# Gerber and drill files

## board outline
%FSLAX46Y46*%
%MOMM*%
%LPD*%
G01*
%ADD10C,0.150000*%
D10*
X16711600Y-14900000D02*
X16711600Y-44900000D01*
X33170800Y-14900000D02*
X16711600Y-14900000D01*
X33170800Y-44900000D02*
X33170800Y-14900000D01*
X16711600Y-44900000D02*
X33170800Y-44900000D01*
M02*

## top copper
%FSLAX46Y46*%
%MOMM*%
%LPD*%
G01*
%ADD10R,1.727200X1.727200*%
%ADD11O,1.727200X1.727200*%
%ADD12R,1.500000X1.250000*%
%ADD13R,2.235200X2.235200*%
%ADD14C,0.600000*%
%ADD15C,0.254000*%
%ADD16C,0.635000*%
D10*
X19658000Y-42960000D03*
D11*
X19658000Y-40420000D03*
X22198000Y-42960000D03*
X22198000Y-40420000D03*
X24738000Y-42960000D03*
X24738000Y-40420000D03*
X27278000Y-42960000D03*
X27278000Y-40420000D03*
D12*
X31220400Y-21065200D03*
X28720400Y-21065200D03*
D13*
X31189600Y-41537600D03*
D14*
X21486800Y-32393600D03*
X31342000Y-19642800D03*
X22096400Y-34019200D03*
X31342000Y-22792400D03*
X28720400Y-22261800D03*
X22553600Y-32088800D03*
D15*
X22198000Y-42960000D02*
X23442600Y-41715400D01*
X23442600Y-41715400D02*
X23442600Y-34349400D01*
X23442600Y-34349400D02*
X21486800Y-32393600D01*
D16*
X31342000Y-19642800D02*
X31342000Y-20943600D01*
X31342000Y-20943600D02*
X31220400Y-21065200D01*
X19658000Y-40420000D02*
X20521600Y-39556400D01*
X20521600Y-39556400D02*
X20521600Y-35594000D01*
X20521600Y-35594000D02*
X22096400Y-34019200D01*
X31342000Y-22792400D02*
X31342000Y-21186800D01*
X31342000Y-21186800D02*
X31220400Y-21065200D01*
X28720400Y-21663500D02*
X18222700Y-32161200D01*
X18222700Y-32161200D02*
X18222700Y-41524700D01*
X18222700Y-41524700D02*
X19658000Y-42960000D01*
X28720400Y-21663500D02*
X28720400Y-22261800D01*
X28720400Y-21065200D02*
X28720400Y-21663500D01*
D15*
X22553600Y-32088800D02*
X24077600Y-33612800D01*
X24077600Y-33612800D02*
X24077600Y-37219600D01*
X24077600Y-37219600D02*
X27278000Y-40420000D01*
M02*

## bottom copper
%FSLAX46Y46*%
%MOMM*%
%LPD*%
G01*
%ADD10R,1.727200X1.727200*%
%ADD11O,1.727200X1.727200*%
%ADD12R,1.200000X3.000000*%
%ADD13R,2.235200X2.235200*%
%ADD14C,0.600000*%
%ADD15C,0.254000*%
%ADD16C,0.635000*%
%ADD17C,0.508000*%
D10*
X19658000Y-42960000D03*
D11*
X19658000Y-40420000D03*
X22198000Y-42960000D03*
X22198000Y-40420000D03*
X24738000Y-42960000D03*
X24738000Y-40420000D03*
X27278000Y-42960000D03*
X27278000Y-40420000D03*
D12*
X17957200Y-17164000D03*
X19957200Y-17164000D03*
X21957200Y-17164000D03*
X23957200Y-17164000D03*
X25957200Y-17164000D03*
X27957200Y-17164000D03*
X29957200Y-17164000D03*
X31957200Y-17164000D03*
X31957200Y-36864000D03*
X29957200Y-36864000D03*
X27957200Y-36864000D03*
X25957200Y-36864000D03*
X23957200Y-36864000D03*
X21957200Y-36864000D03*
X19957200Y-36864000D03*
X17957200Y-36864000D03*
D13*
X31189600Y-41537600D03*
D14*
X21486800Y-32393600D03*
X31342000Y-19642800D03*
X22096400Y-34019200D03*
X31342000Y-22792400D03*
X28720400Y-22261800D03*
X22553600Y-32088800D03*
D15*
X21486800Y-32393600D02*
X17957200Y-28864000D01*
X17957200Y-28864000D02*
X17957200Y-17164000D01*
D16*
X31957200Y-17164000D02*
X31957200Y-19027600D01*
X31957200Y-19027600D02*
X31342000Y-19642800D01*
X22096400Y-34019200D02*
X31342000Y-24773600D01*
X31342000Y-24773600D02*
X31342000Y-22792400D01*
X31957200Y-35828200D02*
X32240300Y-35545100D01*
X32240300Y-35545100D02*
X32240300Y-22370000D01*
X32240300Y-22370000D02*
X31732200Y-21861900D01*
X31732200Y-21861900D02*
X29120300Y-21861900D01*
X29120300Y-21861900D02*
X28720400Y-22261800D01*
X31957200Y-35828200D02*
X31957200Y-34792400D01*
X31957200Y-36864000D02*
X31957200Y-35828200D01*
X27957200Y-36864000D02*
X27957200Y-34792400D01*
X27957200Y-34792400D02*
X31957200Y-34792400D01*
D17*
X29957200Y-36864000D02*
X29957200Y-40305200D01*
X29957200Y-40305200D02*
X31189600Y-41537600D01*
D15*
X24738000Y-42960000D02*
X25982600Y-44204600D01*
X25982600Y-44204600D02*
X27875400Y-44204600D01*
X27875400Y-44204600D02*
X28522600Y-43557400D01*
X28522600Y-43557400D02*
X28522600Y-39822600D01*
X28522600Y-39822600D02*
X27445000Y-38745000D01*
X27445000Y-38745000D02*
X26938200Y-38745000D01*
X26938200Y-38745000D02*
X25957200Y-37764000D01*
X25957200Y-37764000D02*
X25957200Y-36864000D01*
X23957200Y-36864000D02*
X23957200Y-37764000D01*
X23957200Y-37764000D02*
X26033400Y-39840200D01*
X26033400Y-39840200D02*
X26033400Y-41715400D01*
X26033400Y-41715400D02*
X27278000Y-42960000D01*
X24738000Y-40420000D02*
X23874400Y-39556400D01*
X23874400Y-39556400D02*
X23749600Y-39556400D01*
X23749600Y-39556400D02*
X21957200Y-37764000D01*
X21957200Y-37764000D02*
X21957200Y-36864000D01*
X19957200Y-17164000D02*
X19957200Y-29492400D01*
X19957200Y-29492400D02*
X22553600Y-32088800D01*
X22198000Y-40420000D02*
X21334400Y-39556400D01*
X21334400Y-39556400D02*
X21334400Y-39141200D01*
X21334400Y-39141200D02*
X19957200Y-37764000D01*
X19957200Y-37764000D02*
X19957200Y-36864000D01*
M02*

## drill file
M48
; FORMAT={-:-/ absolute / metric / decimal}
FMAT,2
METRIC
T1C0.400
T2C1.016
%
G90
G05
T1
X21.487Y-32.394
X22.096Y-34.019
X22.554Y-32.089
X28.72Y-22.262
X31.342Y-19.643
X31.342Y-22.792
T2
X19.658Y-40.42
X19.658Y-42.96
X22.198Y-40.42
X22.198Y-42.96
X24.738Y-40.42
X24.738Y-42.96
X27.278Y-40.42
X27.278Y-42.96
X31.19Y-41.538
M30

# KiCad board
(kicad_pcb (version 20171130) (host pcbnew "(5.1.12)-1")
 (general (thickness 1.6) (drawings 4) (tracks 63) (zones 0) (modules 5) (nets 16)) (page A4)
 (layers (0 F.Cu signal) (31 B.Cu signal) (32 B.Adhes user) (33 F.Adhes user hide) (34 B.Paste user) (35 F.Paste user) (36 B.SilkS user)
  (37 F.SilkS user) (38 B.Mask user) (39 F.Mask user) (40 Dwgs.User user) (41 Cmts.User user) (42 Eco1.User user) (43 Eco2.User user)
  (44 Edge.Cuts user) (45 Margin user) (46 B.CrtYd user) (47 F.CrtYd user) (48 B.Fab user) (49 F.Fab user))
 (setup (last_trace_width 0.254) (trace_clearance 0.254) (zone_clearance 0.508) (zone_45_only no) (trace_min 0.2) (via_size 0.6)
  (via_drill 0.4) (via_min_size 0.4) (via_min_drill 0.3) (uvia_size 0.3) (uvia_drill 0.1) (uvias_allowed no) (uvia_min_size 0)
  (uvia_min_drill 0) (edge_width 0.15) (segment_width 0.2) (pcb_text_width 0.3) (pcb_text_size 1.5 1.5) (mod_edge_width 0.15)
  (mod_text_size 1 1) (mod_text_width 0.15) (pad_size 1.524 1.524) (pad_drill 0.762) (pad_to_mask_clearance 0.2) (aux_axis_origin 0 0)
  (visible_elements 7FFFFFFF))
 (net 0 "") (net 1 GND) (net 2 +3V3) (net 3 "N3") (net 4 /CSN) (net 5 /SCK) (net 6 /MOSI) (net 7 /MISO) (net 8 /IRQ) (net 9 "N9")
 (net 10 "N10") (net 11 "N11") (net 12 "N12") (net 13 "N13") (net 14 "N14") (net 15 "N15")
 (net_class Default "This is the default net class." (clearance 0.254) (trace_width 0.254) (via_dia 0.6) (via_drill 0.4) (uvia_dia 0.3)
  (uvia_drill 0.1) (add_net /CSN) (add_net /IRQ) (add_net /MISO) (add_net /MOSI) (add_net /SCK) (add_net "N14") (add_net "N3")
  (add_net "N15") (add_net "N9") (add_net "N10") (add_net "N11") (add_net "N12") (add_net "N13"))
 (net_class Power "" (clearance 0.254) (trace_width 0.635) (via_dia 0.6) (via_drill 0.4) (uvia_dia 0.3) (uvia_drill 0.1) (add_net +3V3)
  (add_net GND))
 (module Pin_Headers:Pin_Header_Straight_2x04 (layer F.Cu) (at 19.658 42.96 90)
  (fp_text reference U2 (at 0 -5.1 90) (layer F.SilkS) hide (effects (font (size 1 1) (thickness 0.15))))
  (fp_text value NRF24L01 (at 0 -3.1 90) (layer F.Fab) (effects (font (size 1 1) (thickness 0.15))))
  (pad 1 thru_hole rect (at 0 0 90) (size 1.7272 1.7272) (drill 1.016) (layers *.Cu *.Mask F.SilkS) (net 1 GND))
  (pad 2 thru_hole oval (at 2.54 0 90) (size 1.7272 1.7272) (drill 1.016) (layers *.Cu *.Mask F.SilkS) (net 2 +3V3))
  (pad 3 thru_hole oval (at 0 2.54 90) (size 1.7272 1.7272) (drill 1.016) (layers *.Cu *.Mask F.SilkS) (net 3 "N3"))
  (pad 4 thru_hole oval (at 2.54 2.54 90) (size 1.7272 1.7272) (drill 1.016) (layers *.Cu *.Mask F.SilkS) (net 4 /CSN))
  (pad 5 thru_hole oval (at 0 5.08 90) (size 1.7272 1.7272) (drill 1.016) (layers *.Cu *.Mask F.SilkS) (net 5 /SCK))
  (pad 6 thru_hole oval (at 2.54 5.08 90) (size 1.7272 1.7272) (drill 1.016) (layers *.Cu *.Mask F.SilkS) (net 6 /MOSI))
  (pad 7 thru_hole oval (at 0 7.62 90) (size 1.7272 1.7272) (drill 1.016) (layers *.Cu *.Mask F.SilkS) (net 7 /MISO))
  (pad 8 thru_hole oval (at 2.54 7.62 90) (size 1.7272 1.7272) (drill 1.016) (layers *.Cu *.Mask F.SilkS) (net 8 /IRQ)))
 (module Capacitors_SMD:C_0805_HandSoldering (layer F.Cu) (at 29.9704 21.0652 180)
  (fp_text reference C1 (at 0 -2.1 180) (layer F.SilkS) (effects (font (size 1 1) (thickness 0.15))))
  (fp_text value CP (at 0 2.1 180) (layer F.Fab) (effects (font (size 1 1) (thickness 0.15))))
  (pad 1 smd rect (at -1.25 0 180) (size 1.5 1.25) (layers F.Cu F.Paste F.Mask) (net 2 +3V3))
  (pad 2 smd rect (at 1.25 0 180) (size 1.5 1.25) (layers F.Cu F.Paste F.Mask) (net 1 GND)))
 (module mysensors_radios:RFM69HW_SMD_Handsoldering (layer B.Cu) (at 17.9572 18.564 270)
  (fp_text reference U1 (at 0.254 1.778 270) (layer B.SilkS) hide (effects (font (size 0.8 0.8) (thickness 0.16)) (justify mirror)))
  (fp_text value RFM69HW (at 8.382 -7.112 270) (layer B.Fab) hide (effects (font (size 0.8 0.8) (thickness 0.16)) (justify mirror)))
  (pad 1 smd rect (at -1.4 0 270) (size 3 1.2) (layers B.Cu B.Paste B.Mask) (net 3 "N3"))
  (pad 2 smd rect (at -1.4 -2 270) (size 3 1.2) (layers B.Cu B.Paste B.Mask) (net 8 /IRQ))
  (pad 3 smd rect (at -1.4 -4 270) (size 3 1.2) (layers B.Cu B.Paste B.Mask) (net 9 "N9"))
  (pad 4 smd rect (at -1.4 -6 270) (size 3 1.2) (layers B.Cu B.Paste B.Mask) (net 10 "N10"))
  (pad 5 smd rect (at -1.4 -8 270) (size 3 1.2) (layers B.Cu B.Paste B.Mask) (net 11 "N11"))
  (pad 6 smd rect (at -1.4 -10 270) (size 3 1.2) (layers B.Cu B.Paste B.Mask) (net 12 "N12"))
  (pad 7 smd rect (at -1.4 -12 270) (size 3 1.2) (layers B.Cu B.Paste B.Mask) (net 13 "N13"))
  (pad 8 smd rect (at -1.4 -14 270) (size 3 1.2) (layers B.Cu B.Paste B.Mask) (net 2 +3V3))
  (pad 9 smd rect (at 18.3 -14 270) (size 3 1.2) (layers B.Cu B.Paste B.Mask) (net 1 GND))
  (pad 10 smd rect (at 18.3 -12 270) (size 3 1.2) (layers B.Cu B.Paste B.Mask) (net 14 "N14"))
  (pad 11 smd rect (at 18.3 -10 270) (size 3 1.2) (layers B.Cu B.Paste B.Mask) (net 1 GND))
  (pad 12 smd rect (at 18.3 -8 270) (size 3 1.2) (layers B.Cu B.Paste B.Mask) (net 5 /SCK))
  (pad 13 smd rect (at 18.3 -6 270) (size 3 1.2) (layers B.Cu B.Paste B.Mask) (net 7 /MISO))
  (pad 14 smd rect (at 18.3 -4 270) (size 3 1.2) (layers B.Cu B.Paste B.Mask) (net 6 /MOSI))
  (pad 15 smd rect (at 18.3 -2 270) (size 3 1.2) (layers B.Cu B.Paste B.Mask) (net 4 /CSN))
  (pad 16 smd rect (at 18.3 0 270) (size 3 1.2) (layers B.Cu B.Paste B.Mask) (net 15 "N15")))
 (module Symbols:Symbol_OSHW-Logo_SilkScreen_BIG (layer F.Cu) (at 24.6872 8.7716)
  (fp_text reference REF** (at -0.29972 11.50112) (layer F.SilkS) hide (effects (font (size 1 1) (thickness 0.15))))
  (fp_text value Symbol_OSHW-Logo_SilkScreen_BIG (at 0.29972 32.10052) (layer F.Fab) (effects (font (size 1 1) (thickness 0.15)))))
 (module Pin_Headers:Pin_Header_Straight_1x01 (layer F.Cu) (at 31.1896 41.5376)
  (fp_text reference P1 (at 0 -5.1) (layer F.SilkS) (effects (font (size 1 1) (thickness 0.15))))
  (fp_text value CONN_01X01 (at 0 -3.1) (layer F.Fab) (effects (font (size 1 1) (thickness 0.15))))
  (pad 1 thru_hole rect (at 0 0) (size 2.2352 2.2352) (drill 1.016) (layers *.Cu *.Mask F.SilkS) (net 14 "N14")))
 (gr_line (start 16.7116 14.9) (end 16.7116 44.9) (layer Edge.Cuts) (width 0.15))
 (gr_line (start 33.1708 14.9) (end 16.7116 14.9) (layer Edge.Cuts) (width 0.15))
 (gr_line (start 33.1708 44.9) (end 33.1708 14.9) (layer Edge.Cuts) (width 0.15))
 (gr_line (start 16.7116 44.9) (end 33.1708 44.9) (layer Edge.Cuts) (width 0.15))
 (segment (start 22.198 42.96) (end 23.4426 41.7154) (width 0.254) (layer F.Cu) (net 3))
 (segment (start 23.4426 41.7154) (end 23.4426 34.3494) (width 0.254) (layer F.Cu) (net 3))
 (segment (start 23.4426 34.3494) (end 21.4868 32.3936) (width 0.254) (layer F.Cu) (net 3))
 (segment (start 21.4868 32.3936) (end 17.9572 28.864) (width 0.254) (layer B.Cu) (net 3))
 (segment (start 17.9572 28.864) (end 17.9572 17.164) (width 0.254) (layer B.Cu) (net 3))
 (via (at 21.4868 32.3936) (size 0.6) (layers F.Cu B.Cu) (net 3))
 (segment (start 31.9572 17.164) (end 31.9572 19.0276) (width 0.635) (layer B.Cu) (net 2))
 (segment (start 31.9572 19.0276) (end 31.342 19.6428) (width 0.635) (layer B.Cu) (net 2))
 (segment (start 31.342 19.6428) (end 31.342 20.9436) (width 0.635) (layer F.Cu) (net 2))
 (segment (start 31.342 20.9436) (end 31.2204 21.0652) (width 0.635) (layer F.Cu) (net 2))
 (segment (start 19.658 40.42) (end 20.5216 39.5564) (width 0.635) (layer F.Cu) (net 2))
 (segment (start 20.5216 39.5564) (end 20.5216 35.594) (width 0.635) (layer F.Cu) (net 2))
 (segment (start 20.5216 35.594) (end 22.0964 34.0192) (width 0.635) (layer F.Cu) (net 2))
 (segment (start 22.0964 34.0192) (end 31.342 24.7736) (width 0.635) (layer B.Cu) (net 2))
 (segment (start 31.342 24.7736) (end 31.342 22.7924) (width 0.635) (layer B.Cu) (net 2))
 (segment (start 31.342 22.7924) (end 31.342 21.1868) (width 0.635) (layer F.Cu) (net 2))
 (segment (start 31.342 21.1868) (end 31.2204 21.0652) (width 0.635) (layer F.Cu) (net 2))
 (via (at 31.342 19.6428) (size 0.6) (layers F.Cu B.Cu) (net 2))
 (via (at 22.0964 34.0192) (size 0.6) (layers F.Cu B.Cu) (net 2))
 (via (at 31.342 22.7924) (size 0.6) (layers F.Cu B.Cu) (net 2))
 (segment (start 28.7204 21.6635) (end 18.2227 32.1612) (width 0.635) (layer F.Cu) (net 1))
 (segment (start 18.2227 32.1612) (end 18.2227 41.5247) (width 0.635) (layer F.Cu) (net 1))
 (segment (start 18.2227 41.5247) (end 19.658 42.96) (width 0.635) (layer F.Cu) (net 1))
 (segment (start 28.7204 21.6635) (end 28.7204 22.2618) (width 0.635) (layer F.Cu) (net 1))
 (segment (start 28.7204 21.0652) (end 28.7204 21.6635) (width 0.635) (layer F.Cu) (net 1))
 (segment (start 31.9572 35.8282) (end 32.2403 35.5451) (width 0.635) (layer B.Cu) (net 1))
 (segment (start 32.2403 35.5451) (end 32.2403 22.37) (width 0.635) (layer B.Cu) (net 1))
 (segment (start 32.2403 22.37) (end 31.7322 21.8619) (width 0.635) (layer B.Cu) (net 1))
 (segment (start 31.7322 21.8619) (end 29.1203 21.8619) (width 0.635) (layer B.Cu) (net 1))
 (segment (start 29.1203 21.8619) (end 28.7204 22.2618) (width 0.635) (layer B.Cu) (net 1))
 (segment (start 31.9572 35.8282) (end 31.9572 34.7924) (width 0.635) (layer B.Cu) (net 1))
 (segment (start 31.9572 36.864) (end 31.9572 35.8282) (width 0.635) (layer B.Cu) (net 1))
 (segment (start 27.9572 36.864) (end 27.9572 34.7924) (width 0.635) (layer B.Cu) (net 1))
 (segment (start 27.9572 34.7924) (end 31.9572 34.7924) (width 0.635) (layer B.Cu) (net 1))
 (via (at 28.7204 22.2618) (size 0.6) (layers F.Cu B.Cu) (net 1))
 (segment (start 29.9572 36.864) (end 29.9572 40.3052) (width 0.508) (layer B.Cu) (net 14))
 (segment (start 29.9572 40.3052) (end 31.1896 41.5376) (width 0.508) (layer B.Cu) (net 14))
 (segment (start 24.738 42.96) (end 25.9826 44.2046) (width 0.254) (layer B.Cu) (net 5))
 (segment (start 25.9826 44.2046) (end 27.8754 44.2046) (width 0.254) (layer B.Cu) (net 5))
 (segment (start 27.8754 44.2046) (end 28.5226 43.5574) (width 0.254) (layer B.Cu) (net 5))
 (segment (start 28.5226 43.5574) (end 28.5226 39.8226) (width 0.254) (layer B.Cu) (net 5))
 (segment (start 28.5226 39.8226) (end 27.445 38.745) (width 0.254) (layer B.Cu) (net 5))
 (segment (start 27.445 38.745) (end 26.9382 38.745) (width 0.254) (layer B.Cu) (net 5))
 (segment (start 26.9382 38.745) (end 25.9572 37.764) (width 0.254) (layer B.Cu) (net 5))
 (segment (start 25.9572 37.764) (end 25.9572 36.864) (width 0.254) (layer B.Cu) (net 5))
 (segment (start 23.9572 36.864) (end 23.9572 37.764) (width 0.254) (layer B.Cu) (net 7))
 (segment (start 23.9572 37.764) (end 26.0334 39.8402) (width 0.254) (layer B.Cu) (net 7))
 (segment (start 26.0334 39.8402) (end 26.0334 41.7154) (width 0.254) (layer B.Cu) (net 7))
 (segment (start 26.0334 41.7154) (end 27.278 42.96) (width 0.254) (layer B.Cu) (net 7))
 (segment (start 24.738 40.42) (end 23.8744 39.5564) (width 0.254) (layer B.Cu) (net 6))
 (segment (start 23.8744 39.5564) (end 23.7496 39.5564) (width 0.254) (layer B.Cu) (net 6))
 (segment (start 23.7496 39.5564) (end 21.9572 37.764) (width 0.254) (layer B.Cu) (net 6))
 (segment (start 21.9572 37.764) (end 21.9572 36.864) (width 0.254) (layer B.Cu) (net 6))
 (segment (start 19.9572 17.164) (end 19.9572 29.4924) (width 0.254) (layer B.Cu) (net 8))
 (segment (start 19.9572 29.4924) (end 22.5536 32.0888) (width 0.254) (layer B.Cu) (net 8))
 (segment (start 22.5536 32.0888) (end 24.0776 33.6128) (width 0.254) (layer F.Cu) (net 8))
 (segment (start 24.0776 33.6128) (end 24.0776 37.2196) (width 0.254) (layer F.Cu) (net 8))
 (segment (start 24.0776 37.2196) (end 27.278 40.42) (width 0.254) (layer F.Cu) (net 8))
 (via (at 22.5536 32.0888) (size 0.6) (layers F.Cu B.Cu) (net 8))
 (segment (start 22.198 40.42) (end 21.3344 39.5564) (width 0.254) (layer B.Cu) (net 4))
 (segment (start 21.3344 39.5564) (end 21.3344 39.1412) (width 0.254) (layer B.Cu) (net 4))
 (segment (start 21.3344 39.1412) (end 19.9572 37.764) (width 0.254) (layer B.Cu) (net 4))
 (segment (start 19.9572 37.764) (end 19.9572 36.864) (width 0.254) (layer B.Cu) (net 4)))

